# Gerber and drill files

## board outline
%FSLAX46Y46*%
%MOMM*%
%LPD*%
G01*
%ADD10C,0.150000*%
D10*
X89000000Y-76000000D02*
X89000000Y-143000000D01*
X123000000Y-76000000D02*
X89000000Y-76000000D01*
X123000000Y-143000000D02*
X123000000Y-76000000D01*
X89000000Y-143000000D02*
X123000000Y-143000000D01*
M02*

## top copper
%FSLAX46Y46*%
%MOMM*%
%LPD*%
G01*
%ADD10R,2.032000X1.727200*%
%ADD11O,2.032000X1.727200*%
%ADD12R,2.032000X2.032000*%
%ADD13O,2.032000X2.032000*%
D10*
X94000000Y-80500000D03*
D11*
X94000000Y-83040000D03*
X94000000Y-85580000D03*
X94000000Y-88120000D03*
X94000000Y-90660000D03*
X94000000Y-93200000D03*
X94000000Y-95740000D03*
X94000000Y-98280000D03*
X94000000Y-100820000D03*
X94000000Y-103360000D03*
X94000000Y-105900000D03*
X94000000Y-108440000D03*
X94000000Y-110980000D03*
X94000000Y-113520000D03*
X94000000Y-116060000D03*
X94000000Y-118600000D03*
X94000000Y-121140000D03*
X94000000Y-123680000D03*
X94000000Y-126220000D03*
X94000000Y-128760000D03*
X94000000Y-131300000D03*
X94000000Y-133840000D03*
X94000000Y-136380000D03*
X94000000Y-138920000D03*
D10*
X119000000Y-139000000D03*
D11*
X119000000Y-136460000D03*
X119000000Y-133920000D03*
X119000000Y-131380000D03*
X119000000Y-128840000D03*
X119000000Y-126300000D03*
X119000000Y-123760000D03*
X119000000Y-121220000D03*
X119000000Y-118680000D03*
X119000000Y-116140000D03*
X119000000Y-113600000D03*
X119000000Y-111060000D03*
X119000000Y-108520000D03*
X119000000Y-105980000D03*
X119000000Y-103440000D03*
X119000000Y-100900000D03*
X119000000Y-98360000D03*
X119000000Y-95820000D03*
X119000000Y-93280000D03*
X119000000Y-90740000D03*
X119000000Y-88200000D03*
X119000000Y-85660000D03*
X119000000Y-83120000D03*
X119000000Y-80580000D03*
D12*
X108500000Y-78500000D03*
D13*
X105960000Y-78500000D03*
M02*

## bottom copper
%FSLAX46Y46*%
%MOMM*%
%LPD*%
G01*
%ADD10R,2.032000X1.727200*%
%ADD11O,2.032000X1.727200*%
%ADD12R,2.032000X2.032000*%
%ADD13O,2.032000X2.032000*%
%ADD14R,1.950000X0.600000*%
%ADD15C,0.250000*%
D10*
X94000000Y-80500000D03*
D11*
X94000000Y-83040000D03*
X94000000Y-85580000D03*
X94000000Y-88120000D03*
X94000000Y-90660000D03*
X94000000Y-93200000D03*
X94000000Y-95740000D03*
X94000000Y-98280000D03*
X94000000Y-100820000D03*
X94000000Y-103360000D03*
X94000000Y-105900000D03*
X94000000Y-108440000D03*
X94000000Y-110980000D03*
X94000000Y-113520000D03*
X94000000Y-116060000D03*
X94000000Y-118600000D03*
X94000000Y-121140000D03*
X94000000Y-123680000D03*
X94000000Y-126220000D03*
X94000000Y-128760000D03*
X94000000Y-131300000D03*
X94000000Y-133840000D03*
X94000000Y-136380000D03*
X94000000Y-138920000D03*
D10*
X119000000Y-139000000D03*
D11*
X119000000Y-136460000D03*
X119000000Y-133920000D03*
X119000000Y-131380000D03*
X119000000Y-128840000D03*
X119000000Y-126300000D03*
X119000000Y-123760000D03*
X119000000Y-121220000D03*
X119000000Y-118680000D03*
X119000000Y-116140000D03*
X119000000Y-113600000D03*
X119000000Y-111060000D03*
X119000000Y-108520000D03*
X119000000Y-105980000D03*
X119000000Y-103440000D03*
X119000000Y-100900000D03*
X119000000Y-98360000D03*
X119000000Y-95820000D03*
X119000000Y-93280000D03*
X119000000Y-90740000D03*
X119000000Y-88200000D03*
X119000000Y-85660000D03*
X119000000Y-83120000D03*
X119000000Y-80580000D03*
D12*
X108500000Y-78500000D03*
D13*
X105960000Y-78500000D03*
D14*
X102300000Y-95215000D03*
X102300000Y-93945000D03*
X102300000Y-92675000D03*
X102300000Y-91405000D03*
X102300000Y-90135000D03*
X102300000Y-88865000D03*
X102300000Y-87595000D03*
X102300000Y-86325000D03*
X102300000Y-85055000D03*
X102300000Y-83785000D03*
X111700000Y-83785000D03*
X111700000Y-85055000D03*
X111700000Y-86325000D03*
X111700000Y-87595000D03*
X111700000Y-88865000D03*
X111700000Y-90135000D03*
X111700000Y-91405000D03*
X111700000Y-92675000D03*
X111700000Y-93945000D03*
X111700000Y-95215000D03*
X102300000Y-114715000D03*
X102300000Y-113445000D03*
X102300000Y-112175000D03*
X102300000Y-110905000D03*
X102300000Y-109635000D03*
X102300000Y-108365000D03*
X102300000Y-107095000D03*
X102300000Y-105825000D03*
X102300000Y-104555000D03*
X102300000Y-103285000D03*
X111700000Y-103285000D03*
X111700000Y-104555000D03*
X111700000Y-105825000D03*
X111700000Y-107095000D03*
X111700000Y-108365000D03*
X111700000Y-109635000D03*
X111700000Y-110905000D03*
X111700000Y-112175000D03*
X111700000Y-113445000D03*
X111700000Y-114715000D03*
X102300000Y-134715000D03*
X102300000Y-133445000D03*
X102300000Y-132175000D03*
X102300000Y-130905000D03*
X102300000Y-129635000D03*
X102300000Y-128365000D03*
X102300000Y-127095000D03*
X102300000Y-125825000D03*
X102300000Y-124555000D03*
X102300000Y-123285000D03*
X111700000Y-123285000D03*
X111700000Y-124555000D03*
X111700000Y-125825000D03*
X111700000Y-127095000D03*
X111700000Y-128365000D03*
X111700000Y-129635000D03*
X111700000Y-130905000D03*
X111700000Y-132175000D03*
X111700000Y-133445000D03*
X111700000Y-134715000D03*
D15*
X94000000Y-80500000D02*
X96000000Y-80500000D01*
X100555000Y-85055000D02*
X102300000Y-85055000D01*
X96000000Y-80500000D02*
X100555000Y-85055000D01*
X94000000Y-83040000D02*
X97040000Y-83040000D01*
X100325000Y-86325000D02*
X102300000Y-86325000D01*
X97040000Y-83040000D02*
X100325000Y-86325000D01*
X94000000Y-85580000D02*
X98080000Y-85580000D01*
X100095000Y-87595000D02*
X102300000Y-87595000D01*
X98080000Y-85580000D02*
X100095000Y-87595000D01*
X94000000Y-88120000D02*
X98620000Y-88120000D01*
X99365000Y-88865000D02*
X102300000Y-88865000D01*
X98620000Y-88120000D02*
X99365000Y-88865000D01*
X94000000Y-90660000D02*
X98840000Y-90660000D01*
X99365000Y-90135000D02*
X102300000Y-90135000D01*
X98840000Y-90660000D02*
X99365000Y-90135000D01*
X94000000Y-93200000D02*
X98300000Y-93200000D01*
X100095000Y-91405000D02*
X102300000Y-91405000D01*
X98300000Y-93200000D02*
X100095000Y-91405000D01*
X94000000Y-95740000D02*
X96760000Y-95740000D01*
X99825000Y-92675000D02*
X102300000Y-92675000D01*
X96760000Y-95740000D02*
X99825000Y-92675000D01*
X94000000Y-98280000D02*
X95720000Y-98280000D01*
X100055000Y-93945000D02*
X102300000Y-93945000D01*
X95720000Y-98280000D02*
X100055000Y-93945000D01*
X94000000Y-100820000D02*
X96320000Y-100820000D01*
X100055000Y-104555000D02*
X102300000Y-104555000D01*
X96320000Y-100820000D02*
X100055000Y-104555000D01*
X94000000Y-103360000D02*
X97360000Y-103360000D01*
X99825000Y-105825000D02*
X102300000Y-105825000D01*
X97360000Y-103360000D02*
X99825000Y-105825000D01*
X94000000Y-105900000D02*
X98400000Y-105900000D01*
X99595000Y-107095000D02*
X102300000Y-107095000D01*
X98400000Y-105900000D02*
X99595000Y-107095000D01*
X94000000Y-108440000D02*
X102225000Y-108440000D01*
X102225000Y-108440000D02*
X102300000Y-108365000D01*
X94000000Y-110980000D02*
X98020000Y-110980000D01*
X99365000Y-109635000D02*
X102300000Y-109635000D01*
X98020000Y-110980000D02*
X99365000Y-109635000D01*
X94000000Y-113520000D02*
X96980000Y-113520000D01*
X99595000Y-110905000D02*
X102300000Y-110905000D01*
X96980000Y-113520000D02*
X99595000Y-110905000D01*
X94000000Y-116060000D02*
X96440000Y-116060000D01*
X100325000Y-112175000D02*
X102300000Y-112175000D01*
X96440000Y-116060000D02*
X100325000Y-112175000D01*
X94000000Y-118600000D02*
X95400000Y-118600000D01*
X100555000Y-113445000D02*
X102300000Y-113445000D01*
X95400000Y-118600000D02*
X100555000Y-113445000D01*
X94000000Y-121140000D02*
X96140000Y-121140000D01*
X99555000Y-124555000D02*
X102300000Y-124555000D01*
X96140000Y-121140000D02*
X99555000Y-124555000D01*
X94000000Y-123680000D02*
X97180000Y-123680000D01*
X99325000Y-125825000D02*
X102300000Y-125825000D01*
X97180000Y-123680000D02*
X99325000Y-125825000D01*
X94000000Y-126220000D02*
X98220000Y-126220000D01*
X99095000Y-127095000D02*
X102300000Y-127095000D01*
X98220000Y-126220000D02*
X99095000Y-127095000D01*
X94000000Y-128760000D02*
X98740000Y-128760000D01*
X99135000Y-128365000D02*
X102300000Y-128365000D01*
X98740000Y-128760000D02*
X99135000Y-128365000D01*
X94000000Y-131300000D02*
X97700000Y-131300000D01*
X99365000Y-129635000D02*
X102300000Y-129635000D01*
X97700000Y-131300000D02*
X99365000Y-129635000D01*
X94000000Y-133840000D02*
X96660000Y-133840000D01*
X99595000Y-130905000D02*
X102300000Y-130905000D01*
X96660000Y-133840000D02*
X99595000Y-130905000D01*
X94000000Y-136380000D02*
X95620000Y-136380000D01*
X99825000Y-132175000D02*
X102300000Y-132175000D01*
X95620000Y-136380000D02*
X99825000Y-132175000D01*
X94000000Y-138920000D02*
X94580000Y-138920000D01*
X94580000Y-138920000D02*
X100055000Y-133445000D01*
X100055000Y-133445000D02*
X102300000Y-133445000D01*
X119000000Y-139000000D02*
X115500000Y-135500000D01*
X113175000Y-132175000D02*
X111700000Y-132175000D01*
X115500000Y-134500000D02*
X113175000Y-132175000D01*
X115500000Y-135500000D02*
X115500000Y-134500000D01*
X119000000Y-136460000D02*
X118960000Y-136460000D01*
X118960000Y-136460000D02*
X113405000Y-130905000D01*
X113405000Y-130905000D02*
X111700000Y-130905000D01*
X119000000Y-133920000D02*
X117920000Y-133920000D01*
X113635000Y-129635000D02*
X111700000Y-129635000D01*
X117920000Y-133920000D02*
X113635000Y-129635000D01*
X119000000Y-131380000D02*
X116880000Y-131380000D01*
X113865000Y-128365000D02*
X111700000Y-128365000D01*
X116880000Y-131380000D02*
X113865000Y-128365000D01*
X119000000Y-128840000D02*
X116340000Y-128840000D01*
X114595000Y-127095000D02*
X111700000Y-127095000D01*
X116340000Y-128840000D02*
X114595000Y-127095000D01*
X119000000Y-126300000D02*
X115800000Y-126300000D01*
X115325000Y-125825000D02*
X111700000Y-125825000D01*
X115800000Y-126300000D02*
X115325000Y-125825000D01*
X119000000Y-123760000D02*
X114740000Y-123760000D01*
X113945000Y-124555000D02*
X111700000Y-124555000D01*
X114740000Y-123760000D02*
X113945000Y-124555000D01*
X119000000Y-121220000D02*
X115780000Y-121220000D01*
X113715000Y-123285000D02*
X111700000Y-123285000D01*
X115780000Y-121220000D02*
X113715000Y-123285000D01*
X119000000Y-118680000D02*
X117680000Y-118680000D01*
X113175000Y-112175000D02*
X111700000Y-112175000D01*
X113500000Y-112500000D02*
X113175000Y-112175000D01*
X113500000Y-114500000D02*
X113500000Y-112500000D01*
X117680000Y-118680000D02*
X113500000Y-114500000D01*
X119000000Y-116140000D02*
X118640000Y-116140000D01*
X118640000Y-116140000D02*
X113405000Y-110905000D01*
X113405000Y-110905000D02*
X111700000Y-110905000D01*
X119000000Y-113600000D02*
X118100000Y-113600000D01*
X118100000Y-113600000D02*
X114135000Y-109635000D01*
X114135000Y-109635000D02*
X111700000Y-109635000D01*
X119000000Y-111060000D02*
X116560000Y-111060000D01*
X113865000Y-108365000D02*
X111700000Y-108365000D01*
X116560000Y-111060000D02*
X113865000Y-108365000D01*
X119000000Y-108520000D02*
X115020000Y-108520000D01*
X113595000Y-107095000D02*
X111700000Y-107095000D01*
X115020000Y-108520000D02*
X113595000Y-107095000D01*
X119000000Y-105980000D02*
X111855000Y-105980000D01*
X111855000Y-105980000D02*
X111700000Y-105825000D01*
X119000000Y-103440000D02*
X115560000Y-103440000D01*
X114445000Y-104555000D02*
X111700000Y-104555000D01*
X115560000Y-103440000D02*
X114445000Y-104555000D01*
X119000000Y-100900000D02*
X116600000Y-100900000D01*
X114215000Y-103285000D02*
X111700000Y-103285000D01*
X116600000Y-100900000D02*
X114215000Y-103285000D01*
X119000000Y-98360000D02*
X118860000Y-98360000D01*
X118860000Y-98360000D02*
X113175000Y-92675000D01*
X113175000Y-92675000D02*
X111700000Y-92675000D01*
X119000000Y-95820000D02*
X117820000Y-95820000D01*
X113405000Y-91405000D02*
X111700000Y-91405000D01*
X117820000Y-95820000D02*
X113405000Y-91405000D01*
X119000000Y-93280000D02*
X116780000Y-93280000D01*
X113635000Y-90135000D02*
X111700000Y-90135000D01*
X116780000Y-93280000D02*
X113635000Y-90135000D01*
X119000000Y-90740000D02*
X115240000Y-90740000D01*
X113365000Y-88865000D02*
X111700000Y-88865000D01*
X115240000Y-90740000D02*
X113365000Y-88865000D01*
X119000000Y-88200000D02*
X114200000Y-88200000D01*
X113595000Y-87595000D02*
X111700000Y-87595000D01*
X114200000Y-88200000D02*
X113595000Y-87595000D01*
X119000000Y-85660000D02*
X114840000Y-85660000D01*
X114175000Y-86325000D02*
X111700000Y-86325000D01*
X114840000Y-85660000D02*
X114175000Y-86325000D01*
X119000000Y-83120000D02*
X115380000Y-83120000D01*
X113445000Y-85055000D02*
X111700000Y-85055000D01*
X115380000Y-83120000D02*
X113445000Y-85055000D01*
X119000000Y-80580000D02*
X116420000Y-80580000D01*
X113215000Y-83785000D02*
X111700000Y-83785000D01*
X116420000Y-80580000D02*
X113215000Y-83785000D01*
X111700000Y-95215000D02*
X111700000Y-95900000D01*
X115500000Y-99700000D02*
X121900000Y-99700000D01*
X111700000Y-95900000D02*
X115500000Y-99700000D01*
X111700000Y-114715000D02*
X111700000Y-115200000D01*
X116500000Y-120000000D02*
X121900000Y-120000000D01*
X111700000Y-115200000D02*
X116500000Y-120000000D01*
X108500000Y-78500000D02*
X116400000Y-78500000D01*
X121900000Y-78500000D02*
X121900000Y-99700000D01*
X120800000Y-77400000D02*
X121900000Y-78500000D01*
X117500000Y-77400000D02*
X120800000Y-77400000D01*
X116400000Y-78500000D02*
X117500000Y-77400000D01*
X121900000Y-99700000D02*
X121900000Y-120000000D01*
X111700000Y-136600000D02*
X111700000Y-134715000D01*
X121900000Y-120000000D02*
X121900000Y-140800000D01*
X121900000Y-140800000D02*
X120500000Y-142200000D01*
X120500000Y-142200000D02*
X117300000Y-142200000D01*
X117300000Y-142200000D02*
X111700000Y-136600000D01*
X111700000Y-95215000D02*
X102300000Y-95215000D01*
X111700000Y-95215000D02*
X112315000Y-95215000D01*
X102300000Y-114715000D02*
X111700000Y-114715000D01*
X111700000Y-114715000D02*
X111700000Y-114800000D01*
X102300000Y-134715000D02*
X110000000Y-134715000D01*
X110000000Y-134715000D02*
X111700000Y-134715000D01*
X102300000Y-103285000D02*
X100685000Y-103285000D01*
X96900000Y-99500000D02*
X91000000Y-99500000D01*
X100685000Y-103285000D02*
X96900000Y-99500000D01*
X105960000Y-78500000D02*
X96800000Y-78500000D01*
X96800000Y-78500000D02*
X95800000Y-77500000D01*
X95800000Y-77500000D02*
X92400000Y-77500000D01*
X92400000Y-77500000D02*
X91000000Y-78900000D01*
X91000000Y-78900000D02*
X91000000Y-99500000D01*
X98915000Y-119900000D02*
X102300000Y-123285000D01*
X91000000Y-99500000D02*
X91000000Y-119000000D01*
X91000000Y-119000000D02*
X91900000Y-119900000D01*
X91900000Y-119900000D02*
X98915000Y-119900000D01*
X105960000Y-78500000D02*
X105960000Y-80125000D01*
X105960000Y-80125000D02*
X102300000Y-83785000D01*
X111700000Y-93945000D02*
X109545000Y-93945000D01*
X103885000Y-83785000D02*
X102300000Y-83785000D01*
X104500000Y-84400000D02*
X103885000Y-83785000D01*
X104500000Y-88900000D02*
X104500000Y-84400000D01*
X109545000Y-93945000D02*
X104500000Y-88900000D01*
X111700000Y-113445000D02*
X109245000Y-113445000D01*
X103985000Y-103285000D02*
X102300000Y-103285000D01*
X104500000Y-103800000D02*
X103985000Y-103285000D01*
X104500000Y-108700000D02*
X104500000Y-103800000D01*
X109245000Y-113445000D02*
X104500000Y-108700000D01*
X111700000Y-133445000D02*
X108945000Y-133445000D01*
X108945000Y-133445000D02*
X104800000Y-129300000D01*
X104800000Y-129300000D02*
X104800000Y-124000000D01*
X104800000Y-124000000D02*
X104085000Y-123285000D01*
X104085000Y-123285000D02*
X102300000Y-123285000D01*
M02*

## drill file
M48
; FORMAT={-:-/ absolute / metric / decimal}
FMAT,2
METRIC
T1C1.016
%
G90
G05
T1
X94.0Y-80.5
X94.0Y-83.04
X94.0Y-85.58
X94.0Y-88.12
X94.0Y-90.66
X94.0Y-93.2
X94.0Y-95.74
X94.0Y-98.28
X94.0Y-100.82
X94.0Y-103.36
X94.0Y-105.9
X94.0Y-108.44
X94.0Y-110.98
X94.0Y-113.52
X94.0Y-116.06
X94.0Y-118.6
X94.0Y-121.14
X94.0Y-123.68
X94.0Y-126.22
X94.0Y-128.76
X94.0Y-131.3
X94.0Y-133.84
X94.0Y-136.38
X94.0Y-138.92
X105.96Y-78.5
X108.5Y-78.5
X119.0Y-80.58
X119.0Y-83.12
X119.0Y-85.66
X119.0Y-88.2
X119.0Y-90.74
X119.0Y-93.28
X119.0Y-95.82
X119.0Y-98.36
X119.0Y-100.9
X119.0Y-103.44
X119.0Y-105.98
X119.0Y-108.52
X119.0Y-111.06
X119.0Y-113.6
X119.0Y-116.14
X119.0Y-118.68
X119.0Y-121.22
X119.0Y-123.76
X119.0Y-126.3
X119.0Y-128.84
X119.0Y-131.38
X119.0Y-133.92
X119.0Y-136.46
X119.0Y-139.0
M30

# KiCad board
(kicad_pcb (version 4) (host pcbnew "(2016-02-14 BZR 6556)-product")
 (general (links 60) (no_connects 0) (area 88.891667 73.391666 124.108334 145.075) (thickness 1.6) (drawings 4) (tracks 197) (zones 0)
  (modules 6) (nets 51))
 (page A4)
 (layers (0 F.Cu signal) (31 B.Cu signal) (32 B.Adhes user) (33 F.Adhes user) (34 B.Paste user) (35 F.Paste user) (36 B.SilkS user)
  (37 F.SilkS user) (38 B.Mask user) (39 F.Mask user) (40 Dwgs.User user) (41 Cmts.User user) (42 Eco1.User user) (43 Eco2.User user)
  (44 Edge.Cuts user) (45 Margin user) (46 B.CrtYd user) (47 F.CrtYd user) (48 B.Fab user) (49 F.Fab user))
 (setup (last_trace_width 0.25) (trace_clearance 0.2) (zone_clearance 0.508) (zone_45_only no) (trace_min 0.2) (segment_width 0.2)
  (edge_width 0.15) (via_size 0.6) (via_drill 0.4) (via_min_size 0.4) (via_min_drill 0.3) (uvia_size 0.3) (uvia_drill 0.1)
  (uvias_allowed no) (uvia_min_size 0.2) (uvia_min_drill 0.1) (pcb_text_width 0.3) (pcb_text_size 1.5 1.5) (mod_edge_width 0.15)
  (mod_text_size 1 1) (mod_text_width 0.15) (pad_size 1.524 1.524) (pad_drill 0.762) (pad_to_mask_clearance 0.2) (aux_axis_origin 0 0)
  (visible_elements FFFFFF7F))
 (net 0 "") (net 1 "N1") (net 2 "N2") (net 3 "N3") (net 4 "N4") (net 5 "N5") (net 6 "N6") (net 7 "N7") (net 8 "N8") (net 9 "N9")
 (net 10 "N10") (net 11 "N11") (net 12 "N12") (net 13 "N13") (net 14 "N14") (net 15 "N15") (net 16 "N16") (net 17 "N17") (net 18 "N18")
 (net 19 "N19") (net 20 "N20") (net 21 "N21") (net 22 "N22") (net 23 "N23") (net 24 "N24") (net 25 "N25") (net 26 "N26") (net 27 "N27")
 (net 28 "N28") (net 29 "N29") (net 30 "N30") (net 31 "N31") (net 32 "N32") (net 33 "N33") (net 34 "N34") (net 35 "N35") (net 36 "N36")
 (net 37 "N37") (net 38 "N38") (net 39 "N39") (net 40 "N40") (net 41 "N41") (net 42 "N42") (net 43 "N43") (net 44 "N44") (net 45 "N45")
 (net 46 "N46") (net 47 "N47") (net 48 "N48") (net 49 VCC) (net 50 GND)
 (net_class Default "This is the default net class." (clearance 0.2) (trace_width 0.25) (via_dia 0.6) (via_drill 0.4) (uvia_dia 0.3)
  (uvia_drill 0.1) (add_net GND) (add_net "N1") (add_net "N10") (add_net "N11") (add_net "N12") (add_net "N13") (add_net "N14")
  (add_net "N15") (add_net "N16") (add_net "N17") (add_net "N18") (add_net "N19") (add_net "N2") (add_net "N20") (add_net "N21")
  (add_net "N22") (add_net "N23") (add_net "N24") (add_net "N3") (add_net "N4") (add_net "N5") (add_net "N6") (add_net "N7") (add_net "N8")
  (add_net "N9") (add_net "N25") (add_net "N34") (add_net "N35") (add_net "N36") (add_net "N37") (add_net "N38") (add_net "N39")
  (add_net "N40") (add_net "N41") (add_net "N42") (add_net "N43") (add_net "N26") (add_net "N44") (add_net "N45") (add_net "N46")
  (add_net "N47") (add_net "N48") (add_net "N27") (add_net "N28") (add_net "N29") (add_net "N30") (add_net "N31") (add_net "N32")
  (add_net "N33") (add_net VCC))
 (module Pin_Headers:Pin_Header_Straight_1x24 (layer F.Cu) (at 94 80.5)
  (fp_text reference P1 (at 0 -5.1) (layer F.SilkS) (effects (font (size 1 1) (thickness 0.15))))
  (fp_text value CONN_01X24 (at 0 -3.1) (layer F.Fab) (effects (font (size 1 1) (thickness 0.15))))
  (pad 1 thru_hole rect (at 0 0) (size 2.032 1.7272) (drill 1.016) (layers *.Cu *.Mask F.SilkS) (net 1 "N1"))
  (pad 2 thru_hole oval (at 0 2.54) (size 2.032 1.7272) (drill 1.016) (layers *.Cu *.Mask F.SilkS) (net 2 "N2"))
  (pad 3 thru_hole oval (at 0 5.08) (size 2.032 1.7272) (drill 1.016) (layers *.Cu *.Mask F.SilkS) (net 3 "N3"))
  (pad 4 thru_hole oval (at 0 7.62) (size 2.032 1.7272) (drill 1.016) (layers *.Cu *.Mask F.SilkS) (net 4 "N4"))
  (pad 5 thru_hole oval (at 0 10.16) (size 2.032 1.7272) (drill 1.016) (layers *.Cu *.Mask F.SilkS) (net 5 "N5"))
  (pad 6 thru_hole oval (at 0 12.7) (size 2.032 1.7272) (drill 1.016) (layers *.Cu *.Mask F.SilkS) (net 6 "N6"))
  (pad 7 thru_hole oval (at 0 15.24) (size 2.032 1.7272) (drill 1.016) (layers *.Cu *.Mask F.SilkS) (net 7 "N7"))
  (pad 8 thru_hole oval (at 0 17.78) (size 2.032 1.7272) (drill 1.016) (layers *.Cu *.Mask F.SilkS) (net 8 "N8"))
  (pad 9 thru_hole oval (at 0 20.32) (size 2.032 1.7272) (drill 1.016) (layers *.Cu *.Mask F.SilkS) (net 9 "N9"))
  (pad 10 thru_hole oval (at 0 22.86) (size 2.032 1.7272) (drill 1.016) (layers *.Cu *.Mask F.SilkS) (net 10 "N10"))
  (pad 11 thru_hole oval (at 0 25.4) (size 2.032 1.7272) (drill 1.016) (layers *.Cu *.Mask F.SilkS) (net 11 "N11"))
  (pad 12 thru_hole oval (at 0 27.94) (size 2.032 1.7272) (drill 1.016) (layers *.Cu *.Mask F.SilkS) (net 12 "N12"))
  (pad 13 thru_hole oval (at 0 30.48) (size 2.032 1.7272) (drill 1.016) (layers *.Cu *.Mask F.SilkS) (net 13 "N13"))
  (pad 14 thru_hole oval (at 0 33.02) (size 2.032 1.7272) (drill 1.016) (layers *.Cu *.Mask F.SilkS) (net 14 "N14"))
  (pad 15 thru_hole oval (at 0 35.56) (size 2.032 1.7272) (drill 1.016) (layers *.Cu *.Mask F.SilkS) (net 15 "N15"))
  (pad 16 thru_hole oval (at 0 38.1) (size 2.032 1.7272) (drill 1.016) (layers *.Cu *.Mask F.SilkS) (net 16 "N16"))
  (pad 17 thru_hole oval (at 0 40.64) (size 2.032 1.7272) (drill 1.016) (layers *.Cu *.Mask F.SilkS) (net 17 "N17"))
  (pad 18 thru_hole oval (at 0 43.18) (size 2.032 1.7272) (drill 1.016) (layers *.Cu *.Mask F.SilkS) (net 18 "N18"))
  (pad 19 thru_hole oval (at 0 45.72) (size 2.032 1.7272) (drill 1.016) (layers *.Cu *.Mask F.SilkS) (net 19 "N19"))
  (pad 20 thru_hole oval (at 0 48.26) (size 2.032 1.7272) (drill 1.016) (layers *.Cu *.Mask F.SilkS) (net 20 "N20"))
  (pad 21 thru_hole oval (at 0 50.8) (size 2.032 1.7272) (drill 1.016) (layers *.Cu *.Mask F.SilkS) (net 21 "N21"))
  (pad 22 thru_hole oval (at 0 53.34) (size 2.032 1.7272) (drill 1.016) (layers *.Cu *.Mask F.SilkS) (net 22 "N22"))
  (pad 23 thru_hole oval (at 0 55.88) (size 2.032 1.7272) (drill 1.016) (layers *.Cu *.Mask F.SilkS) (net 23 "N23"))
  (pad 24 thru_hole oval (at 0 58.42) (size 2.032 1.7272) (drill 1.016) (layers *.Cu *.Mask F.SilkS) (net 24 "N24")))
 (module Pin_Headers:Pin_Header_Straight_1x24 (layer F.Cu) (at 119 139 180)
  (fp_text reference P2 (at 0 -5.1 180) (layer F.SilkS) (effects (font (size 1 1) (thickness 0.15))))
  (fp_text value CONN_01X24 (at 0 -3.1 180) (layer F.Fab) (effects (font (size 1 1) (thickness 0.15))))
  (pad 1 thru_hole rect (at 0 0 180) (size 2.032 1.7272) (drill 1.016) (layers *.Cu *.Mask F.SilkS) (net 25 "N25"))
  (pad 2 thru_hole oval (at 0 2.54 180) (size 2.032 1.7272) (drill 1.016) (layers *.Cu *.Mask F.SilkS) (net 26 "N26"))
  (pad 3 thru_hole oval (at 0 5.08 180) (size 2.032 1.7272) (drill 1.016) (layers *.Cu *.Mask F.SilkS) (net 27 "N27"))
  (pad 4 thru_hole oval (at 0 7.62 180) (size 2.032 1.7272) (drill 1.016) (layers *.Cu *.Mask F.SilkS) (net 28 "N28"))
  (pad 5 thru_hole oval (at 0 10.16 180) (size 2.032 1.7272) (drill 1.016) (layers *.Cu *.Mask F.SilkS) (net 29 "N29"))
  (pad 6 thru_hole oval (at 0 12.7 180) (size 2.032 1.7272) (drill 1.016) (layers *.Cu *.Mask F.SilkS) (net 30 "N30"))
  (pad 7 thru_hole oval (at 0 15.24 180) (size 2.032 1.7272) (drill 1.016) (layers *.Cu *.Mask F.SilkS) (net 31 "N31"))
  (pad 8 thru_hole oval (at 0 17.78 180) (size 2.032 1.7272) (drill 1.016) (layers *.Cu *.Mask F.SilkS) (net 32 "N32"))
  (pad 9 thru_hole oval (at 0 20.32 180) (size 2.032 1.7272) (drill 1.016) (layers *.Cu *.Mask F.SilkS) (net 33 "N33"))
  (pad 10 thru_hole oval (at 0 22.86 180) (size 2.032 1.7272) (drill 1.016) (layers *.Cu *.Mask F.SilkS) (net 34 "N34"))
  (pad 11 thru_hole oval (at 0 25.4 180) (size 2.032 1.7272) (drill 1.016) (layers *.Cu *.Mask F.SilkS) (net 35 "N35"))
  (pad 12 thru_hole oval (at 0 27.94 180) (size 2.032 1.7272) (drill 1.016) (layers *.Cu *.Mask F.SilkS) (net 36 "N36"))
  (pad 13 thru_hole oval (at 0 30.48 180) (size 2.032 1.7272) (drill 1.016) (layers *.Cu *.Mask F.SilkS) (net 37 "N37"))
  (pad 14 thru_hole oval (at 0 33.02 180) (size 2.032 1.7272) (drill 1.016) (layers *.Cu *.Mask F.SilkS) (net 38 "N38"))
  (pad 15 thru_hole oval (at 0 35.56 180) (size 2.032 1.7272) (drill 1.016) (layers *.Cu *.Mask F.SilkS) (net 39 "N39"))
  (pad 16 thru_hole oval (at 0 38.1 180) (size 2.032 1.7272) (drill 1.016) (layers *.Cu *.Mask F.SilkS) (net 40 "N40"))
  (pad 17 thru_hole oval (at 0 40.64 180) (size 2.032 1.7272) (drill 1.016) (layers *.Cu *.Mask F.SilkS) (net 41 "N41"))
  (pad 18 thru_hole oval (at 0 43.18 180) (size 2.032 1.7272) (drill 1.016) (layers *.Cu *.Mask F.SilkS) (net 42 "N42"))
  (pad 19 thru_hole oval (at 0 45.72 180) (size 2.032 1.7272) (drill 1.016) (layers *.Cu *.Mask F.SilkS) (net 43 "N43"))
  (pad 20 thru_hole oval (at 0 48.26 180) (size 2.032 1.7272) (drill 1.016) (layers *.Cu *.Mask F.SilkS) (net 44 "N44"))
  (pad 21 thru_hole oval (at 0 50.8 180) (size 2.032 1.7272) (drill 1.016) (layers *.Cu *.Mask F.SilkS) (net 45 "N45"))
  (pad 22 thru_hole oval (at 0 53.34 180) (size 2.032 1.7272) (drill 1.016) (layers *.Cu *.Mask F.SilkS) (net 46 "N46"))
  (pad 23 thru_hole oval (at 0 55.88 180) (size 2.032 1.7272) (drill 1.016) (layers *.Cu *.Mask F.SilkS) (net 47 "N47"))
  (pad 24 thru_hole oval (at 0 58.42 180) (size 2.032 1.7272) (drill 1.016) (layers *.Cu *.Mask F.SilkS) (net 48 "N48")))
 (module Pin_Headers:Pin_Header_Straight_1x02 (layer F.Cu) (at 108.5 78.5 270)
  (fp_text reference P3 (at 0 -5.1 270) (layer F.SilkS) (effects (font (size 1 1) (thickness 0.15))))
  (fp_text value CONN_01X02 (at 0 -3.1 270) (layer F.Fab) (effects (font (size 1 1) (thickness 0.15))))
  (pad 1 thru_hole rect (at 0 0 270) (size 2.032 2.032) (drill 1.016) (layers *.Cu *.Mask F.SilkS) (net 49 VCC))
  (pad 2 thru_hole oval (at 0 2.54 270) (size 2.032 2.032) (drill 1.016) (layers *.Cu *.Mask F.SilkS) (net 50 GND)))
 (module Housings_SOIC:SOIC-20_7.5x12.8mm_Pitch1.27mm (layer B.Cu) (at 107 89.5)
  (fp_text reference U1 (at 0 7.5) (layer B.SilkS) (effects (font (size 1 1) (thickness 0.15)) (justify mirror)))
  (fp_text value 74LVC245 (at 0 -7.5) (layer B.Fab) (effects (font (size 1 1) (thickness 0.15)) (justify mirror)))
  (pad 1 smd rect (at -4.7 5.715) (size 1.95 0.6) (layers B.Cu B.Paste B.Mask) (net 49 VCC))
  (pad 2 smd rect (at -4.7 4.445) (size 1.95 0.6) (layers B.Cu B.Paste B.Mask) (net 8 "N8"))
  (pad 3 smd rect (at -4.7 3.175) (size 1.95 0.6) (layers B.Cu B.Paste B.Mask) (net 7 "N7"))
  (pad 4 smd rect (at -4.7 1.905) (size 1.95 0.6) (layers B.Cu B.Paste B.Mask) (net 6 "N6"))
  (pad 5 smd rect (at -4.7 0.635) (size 1.95 0.6) (layers B.Cu B.Paste B.Mask) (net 5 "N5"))
  (pad 6 smd rect (at -4.7 -0.635) (size 1.95 0.6) (layers B.Cu B.Paste B.Mask) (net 4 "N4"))
  (pad 7 smd rect (at -4.7 -1.905) (size 1.95 0.6) (layers B.Cu B.Paste B.Mask) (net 3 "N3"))
  (pad 8 smd rect (at -4.7 -3.175) (size 1.95 0.6) (layers B.Cu B.Paste B.Mask) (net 2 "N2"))
  (pad 9 smd rect (at -4.7 -4.445) (size 1.95 0.6) (layers B.Cu B.Paste B.Mask) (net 1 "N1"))
  (pad 10 smd rect (at -4.7 -5.715) (size 1.95 0.6) (layers B.Cu B.Paste B.Mask) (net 50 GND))
  (pad 11 smd rect (at 4.7 -5.715) (size 1.95 0.6) (layers B.Cu B.Paste B.Mask) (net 48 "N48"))
  (pad 12 smd rect (at 4.7 -4.445) (size 1.95 0.6) (layers B.Cu B.Paste B.Mask) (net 47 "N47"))
  (pad 13 smd rect (at 4.7 -3.175) (size 1.95 0.6) (layers B.Cu B.Paste B.Mask) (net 46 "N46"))
  (pad 14 smd rect (at 4.7 -1.905) (size 1.95 0.6) (layers B.Cu B.Paste B.Mask) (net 45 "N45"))
  (pad 15 smd rect (at 4.7 -0.635) (size 1.95 0.6) (layers B.Cu B.Paste B.Mask) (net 44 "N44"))
  (pad 16 smd rect (at 4.7 0.635) (size 1.95 0.6) (layers B.Cu B.Paste B.Mask) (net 43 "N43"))
  (pad 17 smd rect (at 4.7 1.905) (size 1.95 0.6) (layers B.Cu B.Paste B.Mask) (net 42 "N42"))
  (pad 18 smd rect (at 4.7 3.175) (size 1.95 0.6) (layers B.Cu B.Paste B.Mask) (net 41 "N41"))
  (pad 19 smd rect (at 4.7 4.445) (size 1.95 0.6) (layers B.Cu B.Paste B.Mask) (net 50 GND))
  (pad 20 smd rect (at 4.7 5.715) (size 1.95 0.6) (layers B.Cu B.Paste B.Mask) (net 49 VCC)))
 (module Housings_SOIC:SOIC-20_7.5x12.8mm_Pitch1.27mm (layer B.Cu) (at 107 109)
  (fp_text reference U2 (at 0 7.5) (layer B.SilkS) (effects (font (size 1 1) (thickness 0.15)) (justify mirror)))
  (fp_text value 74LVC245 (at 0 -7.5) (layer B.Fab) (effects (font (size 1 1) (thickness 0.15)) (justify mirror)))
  (pad 1 smd rect (at -4.7 5.715) (size 1.95 0.6) (layers B.Cu B.Paste B.Mask) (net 49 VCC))
  (pad 2 smd rect (at -4.7 4.445) (size 1.95 0.6) (layers B.Cu B.Paste B.Mask) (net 16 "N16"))
  (pad 3 smd rect (at -4.7 3.175) (size 1.95 0.6) (layers B.Cu B.Paste B.Mask) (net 15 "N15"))
  (pad 4 smd rect (at -4.7 1.905) (size 1.95 0.6) (layers B.Cu B.Paste B.Mask) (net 14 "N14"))
  (pad 5 smd rect (at -4.7 0.635) (size 1.95 0.6) (layers B.Cu B.Paste B.Mask) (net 13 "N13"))
  (pad 6 smd rect (at -4.7 -0.635) (size 1.95 0.6) (layers B.Cu B.Paste B.Mask) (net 12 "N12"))
  (pad 7 smd rect (at -4.7 -1.905) (size 1.95 0.6) (layers B.Cu B.Paste B.Mask) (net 11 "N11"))
  (pad 8 smd rect (at -4.7 -3.175) (size 1.95 0.6) (layers B.Cu B.Paste B.Mask) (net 10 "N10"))
  (pad 9 smd rect (at -4.7 -4.445) (size 1.95 0.6) (layers B.Cu B.Paste B.Mask) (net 9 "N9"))
  (pad 10 smd rect (at -4.7 -5.715) (size 1.95 0.6) (layers B.Cu B.Paste B.Mask) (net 50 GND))
  (pad 11 smd rect (at 4.7 -5.715) (size 1.95 0.6) (layers B.Cu B.Paste B.Mask) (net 40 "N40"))
  (pad 12 smd rect (at 4.7 -4.445) (size 1.95 0.6) (layers B.Cu B.Paste B.Mask) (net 39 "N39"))
  (pad 13 smd rect (at 4.7 -3.175) (size 1.95 0.6) (layers B.Cu B.Paste B.Mask) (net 38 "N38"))
  (pad 14 smd rect (at 4.7 -1.905) (size 1.95 0.6) (layers B.Cu B.Paste B.Mask) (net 37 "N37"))
  (pad 15 smd rect (at 4.7 -0.635) (size 1.95 0.6) (layers B.Cu B.Paste B.Mask) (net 36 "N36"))
  (pad 16 smd rect (at 4.7 0.635) (size 1.95 0.6) (layers B.Cu B.Paste B.Mask) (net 35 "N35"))
  (pad 17 smd rect (at 4.7 1.905) (size 1.95 0.6) (layers B.Cu B.Paste B.Mask) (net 34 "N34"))
  (pad 18 smd rect (at 4.7 3.175) (size 1.95 0.6) (layers B.Cu B.Paste B.Mask) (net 33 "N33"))
  (pad 19 smd rect (at 4.7 4.445) (size 1.95 0.6) (layers B.Cu B.Paste B.Mask) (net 50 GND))
  (pad 20 smd rect (at 4.7 5.715) (size 1.95 0.6) (layers B.Cu B.Paste B.Mask) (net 49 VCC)))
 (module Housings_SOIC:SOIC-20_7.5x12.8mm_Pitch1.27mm (layer B.Cu) (at 107 129)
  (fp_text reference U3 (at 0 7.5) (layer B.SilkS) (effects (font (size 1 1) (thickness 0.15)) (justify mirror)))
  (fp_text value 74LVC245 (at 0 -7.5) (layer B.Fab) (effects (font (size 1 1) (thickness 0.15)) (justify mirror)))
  (pad 1 smd rect (at -4.7 5.715) (size 1.95 0.6) (layers B.Cu B.Paste B.Mask) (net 49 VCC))
  (pad 2 smd rect (at -4.7 4.445) (size 1.95 0.6) (layers B.Cu B.Paste B.Mask) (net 24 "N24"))
  (pad 3 smd rect (at -4.7 3.175) (size 1.95 0.6) (layers B.Cu B.Paste B.Mask) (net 23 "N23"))
  (pad 4 smd rect (at -4.7 1.905) (size 1.95 0.6) (layers B.Cu B.Paste B.Mask) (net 22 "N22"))
  (pad 5 smd rect (at -4.7 0.635) (size 1.95 0.6) (layers B.Cu B.Paste B.Mask) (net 21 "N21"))
  (pad 6 smd rect (at -4.7 -0.635) (size 1.95 0.6) (layers B.Cu B.Paste B.Mask) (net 20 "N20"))
  (pad 7 smd rect (at -4.7 -1.905) (size 1.95 0.6) (layers B.Cu B.Paste B.Mask) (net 19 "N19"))
  (pad 8 smd rect (at -4.7 -3.175) (size 1.95 0.6) (layers B.Cu B.Paste B.Mask) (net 18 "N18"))
  (pad 9 smd rect (at -4.7 -4.445) (size 1.95 0.6) (layers B.Cu B.Paste B.Mask) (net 17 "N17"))
  (pad 10 smd rect (at -4.7 -5.715) (size 1.95 0.6) (layers B.Cu B.Paste B.Mask) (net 50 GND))
  (pad 11 smd rect (at 4.7 -5.715) (size 1.95 0.6) (layers B.Cu B.Paste B.Mask) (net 32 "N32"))
  (pad 12 smd rect (at 4.7 -4.445) (size 1.95 0.6) (layers B.Cu B.Paste B.Mask) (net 31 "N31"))
  (pad 13 smd rect (at 4.7 -3.175) (size 1.95 0.6) (layers B.Cu B.Paste B.Mask) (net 30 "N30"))
  (pad 14 smd rect (at 4.7 -1.905) (size 1.95 0.6) (layers B.Cu B.Paste B.Mask) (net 29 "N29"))
  (pad 15 smd rect (at 4.7 -0.635) (size 1.95 0.6) (layers B.Cu B.Paste B.Mask) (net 28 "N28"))
  (pad 16 smd rect (at 4.7 0.635) (size 1.95 0.6) (layers B.Cu B.Paste B.Mask) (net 27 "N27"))
  (pad 17 smd rect (at 4.7 1.905) (size 1.95 0.6) (layers B.Cu B.Paste B.Mask) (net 26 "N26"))
  (pad 18 smd rect (at 4.7 3.175) (size 1.95 0.6) (layers B.Cu B.Paste B.Mask) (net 25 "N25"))
  (pad 19 smd rect (at 4.7 4.445) (size 1.95 0.6) (layers B.Cu B.Paste B.Mask) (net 50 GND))
  (pad 20 smd rect (at 4.7 5.715) (size 1.95 0.6) (layers B.Cu B.Paste B.Mask) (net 49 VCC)))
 (gr_line (start 89 76) (end 89 143) (angle 90) (layer Edge.Cuts) (width 0.15))
 (gr_line (start 123 76) (end 89 76) (angle 90) (layer Edge.Cuts) (width 0.15))
 (gr_line (start 123 143) (end 123 76) (angle 90) (layer Edge.Cuts) (width 0.15))
 (gr_line (start 89 143) (end 123 143) (angle 90) (layer Edge.Cuts) (width 0.15))
 (segment (start 94 80.5) (end 96 80.5) (width 0.25) (layer B.Cu) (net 1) (status 400000))
 (segment (start 100.555 85.055) (end 102.3 85.055) (width 0.25) (layer B.Cu) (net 1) (status 800000))
 (segment (start 96 80.5) (end 100.555 85.055) (width 0.25) (layer B.Cu) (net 1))
 (segment (start 94 83.04) (end 97.04 83.04) (width 0.25) (layer B.Cu) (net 2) (status 400000))
 (segment (start 100.325 86.325) (end 102.3 86.325) (width 0.25) (layer B.Cu) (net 2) (status 800000))
 (segment (start 97.04 83.04) (end 100.325 86.325) (width 0.25) (layer B.Cu) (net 2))
 (segment (start 94 85.58) (end 98.08 85.58) (width 0.25) (layer B.Cu) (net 3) (status 400000))
 (segment (start 100.095 87.595) (end 102.3 87.595) (width 0.25) (layer B.Cu) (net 3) (status 800000))
 (segment (start 98.08 85.58) (end 100.095 87.595) (width 0.25) (layer B.Cu) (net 3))
 (segment (start 94 88.12) (end 98.62 88.12) (width 0.25) (layer B.Cu) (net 4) (status 400000))
 (segment (start 99.365 88.865) (end 102.3 88.865) (width 0.25) (layer B.Cu) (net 4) (status 800000))
 (segment (start 98.62 88.12) (end 99.365 88.865) (width 0.25) (layer B.Cu) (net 4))
 (segment (start 94 90.66) (end 98.84 90.66) (width 0.25) (layer B.Cu) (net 5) (status 400000))
 (segment (start 99.365 90.135) (end 102.3 90.135) (width 0.25) (layer B.Cu) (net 5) (status 800000))
 (segment (start 98.84 90.66) (end 99.365 90.135) (width 0.25) (layer B.Cu) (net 5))
 (segment (start 94 93.2) (end 98.3 93.2) (width 0.25) (layer B.Cu) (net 6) (status 400000))
 (segment (start 100.095 91.405) (end 102.3 91.405) (width 0.25) (layer B.Cu) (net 6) (status 800000))
 (segment (start 98.3 93.2) (end 100.095 91.405) (width 0.25) (layer B.Cu) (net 6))
 (segment (start 94 95.74) (end 96.76 95.74) (width 0.25) (layer B.Cu) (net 7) (status 400000))
 (segment (start 99.825 92.675) (end 102.3 92.675) (width 0.25) (layer B.Cu) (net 7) (status 800000))
 (segment (start 96.76 95.74) (end 99.825 92.675) (width 0.25) (layer B.Cu) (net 7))
 (segment (start 94 98.28) (end 95.72 98.28) (width 0.25) (layer B.Cu) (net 8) (status 400000))
 (segment (start 100.055 93.945) (end 102.3 93.945) (width 0.25) (layer B.Cu) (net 8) (status 800000))
 (segment (start 95.72 98.28) (end 100.055 93.945) (width 0.25) (layer B.Cu) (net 8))
 (segment (start 94 100.82) (end 96.32 100.82) (width 0.25) (layer B.Cu) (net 9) (status 400000))
 (segment (start 100.055 104.555) (end 102.3 104.555) (width 0.25) (layer B.Cu) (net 9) (status 800000))
 (segment (start 96.32 100.82) (end 100.055 104.555) (width 0.25) (layer B.Cu) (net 9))
 (segment (start 94 103.36) (end 97.36 103.36) (width 0.25) (layer B.Cu) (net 10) (status 400000))
 (segment (start 99.825 105.825) (end 102.3 105.825) (width 0.25) (layer B.Cu) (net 10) (status 800000))
 (segment (start 97.36 103.36) (end 99.825 105.825) (width 0.25) (layer B.Cu) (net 10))
 (segment (start 94 105.9) (end 98.4 105.9) (width 0.25) (layer B.Cu) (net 11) (status 400000))
 (segment (start 99.595 107.095) (end 102.3 107.095) (width 0.25) (layer B.Cu) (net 11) (status 800000))
 (segment (start 98.4 105.9) (end 99.595 107.095) (width 0.25) (layer B.Cu) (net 11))
 (segment (start 94 108.44) (end 102.225 108.44) (width 0.25) (layer B.Cu) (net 12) (status C00000))
 (segment (start 102.225 108.44) (end 102.3 108.365) (width 0.25) (layer B.Cu) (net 12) (status C00000))
 (segment (start 94 110.98) (end 98.02 110.98) (width 0.25) (layer B.Cu) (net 13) (status 400000))
 (segment (start 99.365 109.635) (end 102.3 109.635) (width 0.25) (layer B.Cu) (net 13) (status 800000))
 (segment (start 98.02 110.98) (end 99.365 109.635) (width 0.25) (layer B.Cu) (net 13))
 (segment (start 94 113.52) (end 96.98 113.52) (width 0.25) (layer B.Cu) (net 14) (status 400000))
 (segment (start 99.595 110.905) (end 102.3 110.905) (width 0.25) (layer B.Cu) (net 14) (status 800000))
 (segment (start 96.98 113.52) (end 99.595 110.905) (width 0.25) (layer B.Cu) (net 14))
 (segment (start 94 116.06) (end 96.44 116.06) (width 0.25) (layer B.Cu) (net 15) (status 400000))
 (segment (start 100.325 112.175) (end 102.3 112.175) (width 0.25) (layer B.Cu) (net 15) (status 800000))
 (segment (start 96.44 116.06) (end 100.325 112.175) (width 0.25) (layer B.Cu) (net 15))
 (segment (start 94 118.6) (end 95.4 118.6) (width 0.25) (layer B.Cu) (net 16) (status 400000))
 (segment (start 100.555 113.445) (end 102.3 113.445) (width 0.25) (layer B.Cu) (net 16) (status 800000))
 (segment (start 95.4 118.6) (end 100.555 113.445) (width 0.25) (layer B.Cu) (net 16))
 (segment (start 94 121.14) (end 96.14 121.14) (width 0.25) (layer B.Cu) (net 17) (status 400000))
 (segment (start 99.555 124.555) (end 102.3 124.555) (width 0.25) (layer B.Cu) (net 17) (status 800000))
 (segment (start 96.14 121.14) (end 99.555 124.555) (width 0.25) (layer B.Cu) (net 17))
 (segment (start 94 123.68) (end 97.18 123.68) (width 0.25) (layer B.Cu) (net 18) (status 400000))
 (segment (start 99.325 125.825) (end 102.3 125.825) (width 0.25) (layer B.Cu) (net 18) (status 800000))
 (segment (start 97.18 123.68) (end 99.325 125.825) (width 0.25) (layer B.Cu) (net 18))
 (segment (start 94 126.22) (end 98.22 126.22) (width 0.25) (layer B.Cu) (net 19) (status 400000))
 (segment (start 99.095 127.095) (end 102.3 127.095) (width 0.25) (layer B.Cu) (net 19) (status 800000))
 (segment (start 98.22 126.22) (end 99.095 127.095) (width 0.25) (layer B.Cu) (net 19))
 (segment (start 94 128.76) (end 98.74 128.76) (width 0.25) (layer B.Cu) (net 20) (status 400000))
 (segment (start 99.135 128.365) (end 102.3 128.365) (width 0.25) (layer B.Cu) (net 20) (status 800000))
 (segment (start 98.74 128.76) (end 99.135 128.365) (width 0.25) (layer B.Cu) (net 20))
 (segment (start 94 131.3) (end 97.7 131.3) (width 0.25) (layer B.Cu) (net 21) (status 400000))
 (segment (start 99.365 129.635) (end 102.3 129.635) (width 0.25) (layer B.Cu) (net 21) (status 800000))
 (segment (start 97.7 131.3) (end 99.365 129.635) (width 0.25) (layer B.Cu) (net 21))
 (segment (start 94 133.84) (end 96.66 133.84) (width 0.25) (layer B.Cu) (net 22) (status 400000))
 (segment (start 99.595 130.905) (end 102.3 130.905) (width 0.25) (layer B.Cu) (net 22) (status 800000))
 (segment (start 96.66 133.84) (end 99.595 130.905) (width 0.25) (layer B.Cu) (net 22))
 (segment (start 94 136.38) (end 95.62 136.38) (width 0.25) (layer B.Cu) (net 23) (status 400000))
 (segment (start 99.825 132.175) (end 102.3 132.175) (width 0.25) (layer B.Cu) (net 23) (status 800000))
 (segment (start 95.62 136.38) (end 99.825 132.175) (width 0.25) (layer B.Cu) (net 23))
 (segment (start 94 138.92) (end 94.58 138.92) (width 0.25) (layer B.Cu) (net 24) (status C00000))
 (segment (start 94.58 138.92) (end 100.055 133.445) (width 0.25) (layer B.Cu) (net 24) (status 400000))
 (segment (start 100.055 133.445) (end 102.3 133.445) (width 0.25) (layer B.Cu) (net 24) (status 800000))
 (segment (start 119 139) (end 115.5 135.5) (width 0.25) (layer B.Cu) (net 25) (status 400000))
 (segment (start 113.175 132.175) (end 111.7 132.175) (width 0.25) (layer B.Cu) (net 25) (status 800000))
 (segment (start 115.5 134.5) (end 113.175 132.175) (width 0.25) (layer B.Cu) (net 25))
 (segment (start 115.5 135.5) (end 115.5 134.5) (width 0.25) (layer B.Cu) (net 25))
 (segment (start 119 136.46) (end 118.96 136.46) (width 0.25) (layer B.Cu) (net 26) (status C00000))
 (segment (start 118.96 136.46) (end 113.405 130.905) (width 0.25) (layer B.Cu) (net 26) (status 400000))
 (segment (start 113.405 130.905) (end 111.7 130.905) (width 0.25) (layer B.Cu) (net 26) (status 800000))
 (segment (start 119 133.92) (end 117.92 133.92) (width 0.25) (layer B.Cu) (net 27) (status 400000))
 (segment (start 113.635 129.635) (end 111.7 129.635) (width 0.25) (layer B.Cu) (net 27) (status 800000))
 (segment (start 117.92 133.92) (end 113.635 129.635) (width 0.25) (layer B.Cu) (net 27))
 (segment (start 119 131.38) (end 116.88 131.38) (width 0.25) (layer B.Cu) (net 28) (status 400000))
 (segment (start 113.865 128.365) (end 111.7 128.365) (width 0.25) (layer B.Cu) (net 28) (status 800000))
 (segment (start 116.88 131.38) (end 113.865 128.365) (width 0.25) (layer B.Cu) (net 28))
 (segment (start 119 128.84) (end 116.34 128.84) (width 0.25) (layer B.Cu) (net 29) (status 400000))
 (segment (start 114.595 127.095) (end 111.7 127.095) (width 0.25) (layer B.Cu) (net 29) (status 800000))
 (segment (start 116.34 128.84) (end 114.595 127.095) (width 0.25) (layer B.Cu) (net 29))
 (segment (start 119 126.3) (end 115.8 126.3) (width 0.25) (layer B.Cu) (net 30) (status 400000))
 (segment (start 115.325 125.825) (end 111.7 125.825) (width 0.25) (layer B.Cu) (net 30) (status 800000))
 (segment (start 115.8 126.3) (end 115.325 125.825) (width 0.25) (layer B.Cu) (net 30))
 (segment (start 119 123.76) (end 114.74 123.76) (width 0.25) (layer B.Cu) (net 31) (status 400000))
 (segment (start 113.945 124.555) (end 111.7 124.555) (width 0.25) (layer B.Cu) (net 31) (status 800000))
 (segment (start 114.74 123.76) (end 113.945 124.555) (width 0.25) (layer B.Cu) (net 31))
 (segment (start 119 121.22) (end 115.78 121.22) (width 0.25) (layer B.Cu) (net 32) (status 400000))
 (segment (start 113.715 123.285) (end 111.7 123.285) (width 0.25) (layer B.Cu) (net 32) (status 800000))
 (segment (start 115.78 121.22) (end 113.715 123.285) (width 0.25) (layer B.Cu) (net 32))
 (segment (start 119 118.68) (end 117.68 118.68) (width 0.25) (layer B.Cu) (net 33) (status 400000))
 (segment (start 113.175 112.175) (end 111.7 112.175) (width 0.25) (layer B.Cu) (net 33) (status 800000))
 (segment (start 113.5 112.5) (end 113.175 112.175) (width 0.25) (layer B.Cu) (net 33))
 (segment (start 113.5 114.5) (end 113.5 112.5) (width 0.25) (layer B.Cu) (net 33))
 (segment (start 117.68 118.68) (end 113.5 114.5) (width 0.25) (layer B.Cu) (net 33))
 (segment (start 119 116.14) (end 118.64 116.14) (width 0.25) (layer B.Cu) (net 34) (status C00000))
 (segment (start 118.64 116.14) (end 113.405 110.905) (width 0.25) (layer B.Cu) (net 34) (status 400000))
 (segment (start 113.405 110.905) (end 111.7 110.905) (width 0.25) (layer B.Cu) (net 34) (status 800000))
 (segment (start 119 113.6) (end 118.1 113.6) (width 0.25) (layer B.Cu) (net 35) (status C00000))
 (segment (start 118.1 113.6) (end 114.135 109.635) (width 0.25) (layer B.Cu) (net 35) (status 400000))
 (segment (start 114.135 109.635) (end 111.7 109.635) (width 0.25) (layer B.Cu) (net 35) (status 800000))
 (segment (start 119 111.06) (end 116.56 111.06) (width 0.25) (layer B.Cu) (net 36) (status 400000))
 (segment (start 113.865 108.365) (end 111.7 108.365) (width 0.25) (layer B.Cu) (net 36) (status 800000))
 (segment (start 116.56 111.06) (end 113.865 108.365) (width 0.25) (layer B.Cu) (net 36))
 (segment (start 119 108.52) (end 115.02 108.52) (width 0.25) (layer B.Cu) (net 37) (status 400000))
 (segment (start 113.595 107.095) (end 111.7 107.095) (width 0.25) (layer B.Cu) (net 37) (status 800000))
 (segment (start 115.02 108.52) (end 113.595 107.095) (width 0.25) (layer B.Cu) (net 37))
 (segment (start 119 105.98) (end 111.855 105.98) (width 0.25) (layer B.Cu) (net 38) (status C00000))
 (segment (start 111.855 105.98) (end 111.7 105.825) (width 0.25) (layer B.Cu) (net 38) (status C00000))
 (segment (start 119 103.44) (end 115.56 103.44) (width 0.25) (layer B.Cu) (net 39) (status 400000))
 (segment (start 114.445 104.555) (end 111.7 104.555) (width 0.25) (layer B.Cu) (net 39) (status 800000))
 (segment (start 115.56 103.44) (end 114.445 104.555) (width 0.25) (layer B.Cu) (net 39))
 (segment (start 119 100.9) (end 116.6 100.9) (width 0.25) (layer B.Cu) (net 40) (status 400000))
 (segment (start 114.215 103.285) (end 111.7 103.285) (width 0.25) (layer B.Cu) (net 40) (status 800000))
 (segment (start 116.6 100.9) (end 114.215 103.285) (width 0.25) (layer B.Cu) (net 40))
 (segment (start 119 98.36) (end 118.86 98.36) (width 0.25) (layer B.Cu) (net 41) (status C00000))
 (segment (start 118.86 98.36) (end 113.175 92.675) (width 0.25) (layer B.Cu) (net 41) (status 400000))
 (segment (start 113.175 92.675) (end 111.7 92.675) (width 0.25) (layer B.Cu) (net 41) (status 800000))
 (segment (start 119 95.82) (end 117.82 95.82) (width 0.25) (layer B.Cu) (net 42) (status 400000))
 (segment (start 113.405 91.405) (end 111.7 91.405) (width 0.25) (layer B.Cu) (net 42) (status 800000))
 (segment (start 117.82 95.82) (end 113.405 91.405) (width 0.25) (layer B.Cu) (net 42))
 (segment (start 119 93.28) (end 116.78 93.28) (width 0.25) (layer B.Cu) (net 43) (status 400000))
 (segment (start 113.635 90.135) (end 111.7 90.135) (width 0.25) (layer B.Cu) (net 43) (status 800000))
 (segment (start 116.78 93.28) (end 113.635 90.135) (width 0.25) (layer B.Cu) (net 43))
 (segment (start 119 90.74) (end 115.24 90.74) (width 0.25) (layer B.Cu) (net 44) (status 400000))
 (segment (start 113.365 88.865) (end 111.7 88.865) (width 0.25) (layer B.Cu) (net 44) (status 800000))
 (segment (start 115.24 90.74) (end 113.365 88.865) (width 0.25) (layer B.Cu) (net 44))
 (segment (start 119 88.2) (end 114.2 88.2) (width 0.25) (layer B.Cu) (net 45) (status 400000))
 (segment (start 113.595 87.595) (end 111.7 87.595) (width 0.25) (layer B.Cu) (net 45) (status 800000))
 (segment (start 114.2 88.2) (end 113.595 87.595) (width 0.25) (layer B.Cu) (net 45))
 (segment (start 119 85.66) (end 114.84 85.66) (width 0.25) (layer B.Cu) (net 46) (status 400000))
 (segment (start 114.175 86.325) (end 111.7 86.325) (width 0.25) (layer B.Cu) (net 46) (status 800000))
 (segment (start 114.84 85.66) (end 114.175 86.325) (width 0.25) (layer B.Cu) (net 46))
 (segment (start 119 83.12) (end 115.38 83.12) (width 0.25) (layer B.Cu) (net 47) (status 400000))
 (segment (start 113.445 85.055) (end 111.7 85.055) (width 0.25) (layer B.Cu) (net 47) (status 800000))
 (segment (start 115.38 83.12) (end 113.445 85.055) (width 0.25) (layer B.Cu) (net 47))
 (segment (start 119 80.58) (end 116.42 80.58) (width 0.25) (layer B.Cu) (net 48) (status 400000))
 (segment (start 113.215 83.785) (end 111.7 83.785) (width 0.25) (layer B.Cu) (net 48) (status 800000))
 (segment (start 116.42 80.58) (end 113.215 83.785) (width 0.25) (layer B.Cu) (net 48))
 (segment (start 111.7 95.215) (end 111.7 95.9) (width 0.25) (layer B.Cu) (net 49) (status 400000))
 (segment (start 115.5 99.7) (end 121.9 99.7) (width 0.25) (layer B.Cu) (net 49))
 (segment (start 111.7 95.9) (end 115.5 99.7) (width 0.25) (layer B.Cu) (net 49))
 (segment (start 111.7 114.715) (end 111.7 115.2) (width 0.25) (layer B.Cu) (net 49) (status 400000))
 (segment (start 116.5 120) (end 121.9 120) (width 0.25) (layer B.Cu) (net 49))
 (segment (start 111.7 115.2) (end 116.5 120) (width 0.25) (layer B.Cu) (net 49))
 (segment (start 108.5 78.5) (end 116.4 78.5) (width 0.25) (layer B.Cu) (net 49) (status 400000))
 (segment (start 121.9 78.5) (end 121.9 99.7) (width 0.25) (layer B.Cu) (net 49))
 (segment (start 120.8 77.4) (end 121.9 78.5) (width 0.25) (layer B.Cu) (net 49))
 (segment (start 117.5 77.4) (end 120.8 77.4) (width 0.25) (layer B.Cu) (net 49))
 (segment (start 116.4 78.5) (end 117.5 77.4) (width 0.25) (layer B.Cu) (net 49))
 (segment (start 121.9 99.7) (end 121.9 120) (width 0.25) (layer B.Cu) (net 49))
 (segment (start 111.7 136.6) (end 111.7 134.715) (width 0.25) (layer B.Cu) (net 49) (status 800000))
 (segment (start 121.9 120) (end 121.9 140.8) (width 0.25) (layer B.Cu) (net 49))
 (segment (start 121.9 140.8) (end 120.5 142.2) (width 0.25) (layer B.Cu) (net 49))
 (segment (start 120.5 142.2) (end 117.3 142.2) (width 0.25) (layer B.Cu) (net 49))
 (segment (start 117.3 142.2) (end 111.7 136.6) (width 0.25) (layer B.Cu) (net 49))
 (segment (start 111.7 95.215) (end 102.3 95.215) (width 0.25) (layer B.Cu) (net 49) (status C00000))
 (segment (start 111.7 95.215) (end 112.315 95.215) (width 0.25) (layer B.Cu) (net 49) (status C00000))
 (segment (start 102.3 114.715) (end 111.7 114.715) (width 0.25) (layer B.Cu) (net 49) (status C00000))
 (segment (start 111.7 114.715) (end 111.7 114.8) (width 0.25) (layer B.Cu) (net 49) (status C00000))
 (segment (start 102.3 134.715) (end 110 134.715) (width 0.25) (layer B.Cu) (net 49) (status 400000))
 (segment (start 110 134.715) (end 111.7 134.715) (width 0.25) (layer B.Cu) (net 49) (status 800000))
 (segment (start 102.3 103.285) (end 100.685 103.285) (width 0.25) (layer B.Cu) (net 50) (status 400000))
 (segment (start 96.9 99.5) (end 91 99.5) (width 0.25) (layer B.Cu) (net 50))
 (segment (start 100.685 103.285) (end 96.9 99.5) (width 0.25) (layer B.Cu) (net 50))
 (segment (start 105.96 78.5) (end 96.8 78.5) (width 0.25) (layer B.Cu) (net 50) (status 400000))
 (segment (start 96.8 78.5) (end 95.8 77.5) (width 0.25) (layer B.Cu) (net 50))
 (segment (start 95.8 77.5) (end 92.4 77.5) (width 0.25) (layer B.Cu) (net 50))
 (segment (start 92.4 77.5) (end 91 78.9) (width 0.25) (layer B.Cu) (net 50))
 (segment (start 91 78.9) (end 91 99.5) (width 0.25) (layer B.Cu) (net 50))
 (segment (start 98.915 119.9) (end 102.3 123.285) (width 0.25) (layer B.Cu) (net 50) (status 800000))
 (segment (start 91 99.5) (end 91 119) (width 0.25) (layer B.Cu) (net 50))
 (segment (start 91 119) (end 91.9 119.9) (width 0.25) (layer B.Cu) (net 50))
 (segment (start 91.9 119.9) (end 98.915 119.9) (width 0.25) (layer B.Cu) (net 50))
 (segment (start 105.96 78.5) (end 105.96 80.125) (width 0.25) (layer B.Cu) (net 50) (status 400000))
 (segment (start 105.96 80.125) (end 102.3 83.785) (width 0.25) (layer B.Cu) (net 50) (status 800000))
 (segment (start 111.7 93.945) (end 109.545 93.945) (width 0.25) (layer B.Cu) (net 50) (status 400000))
 (segment (start 103.885 83.785) (end 102.3 83.785) (width 0.25) (layer B.Cu) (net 50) (status 800000))
 (segment (start 104.5 84.4) (end 103.885 83.785) (width 0.25) (layer B.Cu) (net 50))
 (segment (start 104.5 88.9) (end 104.5 84.4) (width 0.25) (layer B.Cu) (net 50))
 (segment (start 109.545 93.945) (end 104.5 88.9) (width 0.25) (layer B.Cu) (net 50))
 (segment (start 111.7 113.445) (end 109.245 113.445) (width 0.25) (layer B.Cu) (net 50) (status 400000))
 (segment (start 103.985 103.285) (end 102.3 103.285) (width 0.25) (layer B.Cu) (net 50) (status 800000))
 (segment (start 104.5 103.8) (end 103.985 103.285) (width 0.25) (layer B.Cu) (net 50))
 (segment (start 104.5 108.7) (end 104.5 103.8) (width 0.25) (layer B.Cu) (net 50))
 (segment (start 109.245 113.445) (end 104.5 108.7) (width 0.25) (layer B.Cu) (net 50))
 (segment (start 111.7 133.445) (end 108.945 133.445) (width 0.25) (layer B.Cu) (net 50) (status 400000))
 (segment (start 108.945 133.445) (end 104.8 129.3) (width 0.25) (layer B.Cu) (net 50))
 (segment (start 104.8 129.3) (end 104.8 124) (width 0.25) (layer B.Cu) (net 50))
 (segment (start 104.8 124) (end 104.085 123.285) (width 0.25) (layer B.Cu) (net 50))
 (segment (start 104.085 123.285) (end 102.3 123.285) (width 0.25) (layer B.Cu) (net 50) (status 800000)))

